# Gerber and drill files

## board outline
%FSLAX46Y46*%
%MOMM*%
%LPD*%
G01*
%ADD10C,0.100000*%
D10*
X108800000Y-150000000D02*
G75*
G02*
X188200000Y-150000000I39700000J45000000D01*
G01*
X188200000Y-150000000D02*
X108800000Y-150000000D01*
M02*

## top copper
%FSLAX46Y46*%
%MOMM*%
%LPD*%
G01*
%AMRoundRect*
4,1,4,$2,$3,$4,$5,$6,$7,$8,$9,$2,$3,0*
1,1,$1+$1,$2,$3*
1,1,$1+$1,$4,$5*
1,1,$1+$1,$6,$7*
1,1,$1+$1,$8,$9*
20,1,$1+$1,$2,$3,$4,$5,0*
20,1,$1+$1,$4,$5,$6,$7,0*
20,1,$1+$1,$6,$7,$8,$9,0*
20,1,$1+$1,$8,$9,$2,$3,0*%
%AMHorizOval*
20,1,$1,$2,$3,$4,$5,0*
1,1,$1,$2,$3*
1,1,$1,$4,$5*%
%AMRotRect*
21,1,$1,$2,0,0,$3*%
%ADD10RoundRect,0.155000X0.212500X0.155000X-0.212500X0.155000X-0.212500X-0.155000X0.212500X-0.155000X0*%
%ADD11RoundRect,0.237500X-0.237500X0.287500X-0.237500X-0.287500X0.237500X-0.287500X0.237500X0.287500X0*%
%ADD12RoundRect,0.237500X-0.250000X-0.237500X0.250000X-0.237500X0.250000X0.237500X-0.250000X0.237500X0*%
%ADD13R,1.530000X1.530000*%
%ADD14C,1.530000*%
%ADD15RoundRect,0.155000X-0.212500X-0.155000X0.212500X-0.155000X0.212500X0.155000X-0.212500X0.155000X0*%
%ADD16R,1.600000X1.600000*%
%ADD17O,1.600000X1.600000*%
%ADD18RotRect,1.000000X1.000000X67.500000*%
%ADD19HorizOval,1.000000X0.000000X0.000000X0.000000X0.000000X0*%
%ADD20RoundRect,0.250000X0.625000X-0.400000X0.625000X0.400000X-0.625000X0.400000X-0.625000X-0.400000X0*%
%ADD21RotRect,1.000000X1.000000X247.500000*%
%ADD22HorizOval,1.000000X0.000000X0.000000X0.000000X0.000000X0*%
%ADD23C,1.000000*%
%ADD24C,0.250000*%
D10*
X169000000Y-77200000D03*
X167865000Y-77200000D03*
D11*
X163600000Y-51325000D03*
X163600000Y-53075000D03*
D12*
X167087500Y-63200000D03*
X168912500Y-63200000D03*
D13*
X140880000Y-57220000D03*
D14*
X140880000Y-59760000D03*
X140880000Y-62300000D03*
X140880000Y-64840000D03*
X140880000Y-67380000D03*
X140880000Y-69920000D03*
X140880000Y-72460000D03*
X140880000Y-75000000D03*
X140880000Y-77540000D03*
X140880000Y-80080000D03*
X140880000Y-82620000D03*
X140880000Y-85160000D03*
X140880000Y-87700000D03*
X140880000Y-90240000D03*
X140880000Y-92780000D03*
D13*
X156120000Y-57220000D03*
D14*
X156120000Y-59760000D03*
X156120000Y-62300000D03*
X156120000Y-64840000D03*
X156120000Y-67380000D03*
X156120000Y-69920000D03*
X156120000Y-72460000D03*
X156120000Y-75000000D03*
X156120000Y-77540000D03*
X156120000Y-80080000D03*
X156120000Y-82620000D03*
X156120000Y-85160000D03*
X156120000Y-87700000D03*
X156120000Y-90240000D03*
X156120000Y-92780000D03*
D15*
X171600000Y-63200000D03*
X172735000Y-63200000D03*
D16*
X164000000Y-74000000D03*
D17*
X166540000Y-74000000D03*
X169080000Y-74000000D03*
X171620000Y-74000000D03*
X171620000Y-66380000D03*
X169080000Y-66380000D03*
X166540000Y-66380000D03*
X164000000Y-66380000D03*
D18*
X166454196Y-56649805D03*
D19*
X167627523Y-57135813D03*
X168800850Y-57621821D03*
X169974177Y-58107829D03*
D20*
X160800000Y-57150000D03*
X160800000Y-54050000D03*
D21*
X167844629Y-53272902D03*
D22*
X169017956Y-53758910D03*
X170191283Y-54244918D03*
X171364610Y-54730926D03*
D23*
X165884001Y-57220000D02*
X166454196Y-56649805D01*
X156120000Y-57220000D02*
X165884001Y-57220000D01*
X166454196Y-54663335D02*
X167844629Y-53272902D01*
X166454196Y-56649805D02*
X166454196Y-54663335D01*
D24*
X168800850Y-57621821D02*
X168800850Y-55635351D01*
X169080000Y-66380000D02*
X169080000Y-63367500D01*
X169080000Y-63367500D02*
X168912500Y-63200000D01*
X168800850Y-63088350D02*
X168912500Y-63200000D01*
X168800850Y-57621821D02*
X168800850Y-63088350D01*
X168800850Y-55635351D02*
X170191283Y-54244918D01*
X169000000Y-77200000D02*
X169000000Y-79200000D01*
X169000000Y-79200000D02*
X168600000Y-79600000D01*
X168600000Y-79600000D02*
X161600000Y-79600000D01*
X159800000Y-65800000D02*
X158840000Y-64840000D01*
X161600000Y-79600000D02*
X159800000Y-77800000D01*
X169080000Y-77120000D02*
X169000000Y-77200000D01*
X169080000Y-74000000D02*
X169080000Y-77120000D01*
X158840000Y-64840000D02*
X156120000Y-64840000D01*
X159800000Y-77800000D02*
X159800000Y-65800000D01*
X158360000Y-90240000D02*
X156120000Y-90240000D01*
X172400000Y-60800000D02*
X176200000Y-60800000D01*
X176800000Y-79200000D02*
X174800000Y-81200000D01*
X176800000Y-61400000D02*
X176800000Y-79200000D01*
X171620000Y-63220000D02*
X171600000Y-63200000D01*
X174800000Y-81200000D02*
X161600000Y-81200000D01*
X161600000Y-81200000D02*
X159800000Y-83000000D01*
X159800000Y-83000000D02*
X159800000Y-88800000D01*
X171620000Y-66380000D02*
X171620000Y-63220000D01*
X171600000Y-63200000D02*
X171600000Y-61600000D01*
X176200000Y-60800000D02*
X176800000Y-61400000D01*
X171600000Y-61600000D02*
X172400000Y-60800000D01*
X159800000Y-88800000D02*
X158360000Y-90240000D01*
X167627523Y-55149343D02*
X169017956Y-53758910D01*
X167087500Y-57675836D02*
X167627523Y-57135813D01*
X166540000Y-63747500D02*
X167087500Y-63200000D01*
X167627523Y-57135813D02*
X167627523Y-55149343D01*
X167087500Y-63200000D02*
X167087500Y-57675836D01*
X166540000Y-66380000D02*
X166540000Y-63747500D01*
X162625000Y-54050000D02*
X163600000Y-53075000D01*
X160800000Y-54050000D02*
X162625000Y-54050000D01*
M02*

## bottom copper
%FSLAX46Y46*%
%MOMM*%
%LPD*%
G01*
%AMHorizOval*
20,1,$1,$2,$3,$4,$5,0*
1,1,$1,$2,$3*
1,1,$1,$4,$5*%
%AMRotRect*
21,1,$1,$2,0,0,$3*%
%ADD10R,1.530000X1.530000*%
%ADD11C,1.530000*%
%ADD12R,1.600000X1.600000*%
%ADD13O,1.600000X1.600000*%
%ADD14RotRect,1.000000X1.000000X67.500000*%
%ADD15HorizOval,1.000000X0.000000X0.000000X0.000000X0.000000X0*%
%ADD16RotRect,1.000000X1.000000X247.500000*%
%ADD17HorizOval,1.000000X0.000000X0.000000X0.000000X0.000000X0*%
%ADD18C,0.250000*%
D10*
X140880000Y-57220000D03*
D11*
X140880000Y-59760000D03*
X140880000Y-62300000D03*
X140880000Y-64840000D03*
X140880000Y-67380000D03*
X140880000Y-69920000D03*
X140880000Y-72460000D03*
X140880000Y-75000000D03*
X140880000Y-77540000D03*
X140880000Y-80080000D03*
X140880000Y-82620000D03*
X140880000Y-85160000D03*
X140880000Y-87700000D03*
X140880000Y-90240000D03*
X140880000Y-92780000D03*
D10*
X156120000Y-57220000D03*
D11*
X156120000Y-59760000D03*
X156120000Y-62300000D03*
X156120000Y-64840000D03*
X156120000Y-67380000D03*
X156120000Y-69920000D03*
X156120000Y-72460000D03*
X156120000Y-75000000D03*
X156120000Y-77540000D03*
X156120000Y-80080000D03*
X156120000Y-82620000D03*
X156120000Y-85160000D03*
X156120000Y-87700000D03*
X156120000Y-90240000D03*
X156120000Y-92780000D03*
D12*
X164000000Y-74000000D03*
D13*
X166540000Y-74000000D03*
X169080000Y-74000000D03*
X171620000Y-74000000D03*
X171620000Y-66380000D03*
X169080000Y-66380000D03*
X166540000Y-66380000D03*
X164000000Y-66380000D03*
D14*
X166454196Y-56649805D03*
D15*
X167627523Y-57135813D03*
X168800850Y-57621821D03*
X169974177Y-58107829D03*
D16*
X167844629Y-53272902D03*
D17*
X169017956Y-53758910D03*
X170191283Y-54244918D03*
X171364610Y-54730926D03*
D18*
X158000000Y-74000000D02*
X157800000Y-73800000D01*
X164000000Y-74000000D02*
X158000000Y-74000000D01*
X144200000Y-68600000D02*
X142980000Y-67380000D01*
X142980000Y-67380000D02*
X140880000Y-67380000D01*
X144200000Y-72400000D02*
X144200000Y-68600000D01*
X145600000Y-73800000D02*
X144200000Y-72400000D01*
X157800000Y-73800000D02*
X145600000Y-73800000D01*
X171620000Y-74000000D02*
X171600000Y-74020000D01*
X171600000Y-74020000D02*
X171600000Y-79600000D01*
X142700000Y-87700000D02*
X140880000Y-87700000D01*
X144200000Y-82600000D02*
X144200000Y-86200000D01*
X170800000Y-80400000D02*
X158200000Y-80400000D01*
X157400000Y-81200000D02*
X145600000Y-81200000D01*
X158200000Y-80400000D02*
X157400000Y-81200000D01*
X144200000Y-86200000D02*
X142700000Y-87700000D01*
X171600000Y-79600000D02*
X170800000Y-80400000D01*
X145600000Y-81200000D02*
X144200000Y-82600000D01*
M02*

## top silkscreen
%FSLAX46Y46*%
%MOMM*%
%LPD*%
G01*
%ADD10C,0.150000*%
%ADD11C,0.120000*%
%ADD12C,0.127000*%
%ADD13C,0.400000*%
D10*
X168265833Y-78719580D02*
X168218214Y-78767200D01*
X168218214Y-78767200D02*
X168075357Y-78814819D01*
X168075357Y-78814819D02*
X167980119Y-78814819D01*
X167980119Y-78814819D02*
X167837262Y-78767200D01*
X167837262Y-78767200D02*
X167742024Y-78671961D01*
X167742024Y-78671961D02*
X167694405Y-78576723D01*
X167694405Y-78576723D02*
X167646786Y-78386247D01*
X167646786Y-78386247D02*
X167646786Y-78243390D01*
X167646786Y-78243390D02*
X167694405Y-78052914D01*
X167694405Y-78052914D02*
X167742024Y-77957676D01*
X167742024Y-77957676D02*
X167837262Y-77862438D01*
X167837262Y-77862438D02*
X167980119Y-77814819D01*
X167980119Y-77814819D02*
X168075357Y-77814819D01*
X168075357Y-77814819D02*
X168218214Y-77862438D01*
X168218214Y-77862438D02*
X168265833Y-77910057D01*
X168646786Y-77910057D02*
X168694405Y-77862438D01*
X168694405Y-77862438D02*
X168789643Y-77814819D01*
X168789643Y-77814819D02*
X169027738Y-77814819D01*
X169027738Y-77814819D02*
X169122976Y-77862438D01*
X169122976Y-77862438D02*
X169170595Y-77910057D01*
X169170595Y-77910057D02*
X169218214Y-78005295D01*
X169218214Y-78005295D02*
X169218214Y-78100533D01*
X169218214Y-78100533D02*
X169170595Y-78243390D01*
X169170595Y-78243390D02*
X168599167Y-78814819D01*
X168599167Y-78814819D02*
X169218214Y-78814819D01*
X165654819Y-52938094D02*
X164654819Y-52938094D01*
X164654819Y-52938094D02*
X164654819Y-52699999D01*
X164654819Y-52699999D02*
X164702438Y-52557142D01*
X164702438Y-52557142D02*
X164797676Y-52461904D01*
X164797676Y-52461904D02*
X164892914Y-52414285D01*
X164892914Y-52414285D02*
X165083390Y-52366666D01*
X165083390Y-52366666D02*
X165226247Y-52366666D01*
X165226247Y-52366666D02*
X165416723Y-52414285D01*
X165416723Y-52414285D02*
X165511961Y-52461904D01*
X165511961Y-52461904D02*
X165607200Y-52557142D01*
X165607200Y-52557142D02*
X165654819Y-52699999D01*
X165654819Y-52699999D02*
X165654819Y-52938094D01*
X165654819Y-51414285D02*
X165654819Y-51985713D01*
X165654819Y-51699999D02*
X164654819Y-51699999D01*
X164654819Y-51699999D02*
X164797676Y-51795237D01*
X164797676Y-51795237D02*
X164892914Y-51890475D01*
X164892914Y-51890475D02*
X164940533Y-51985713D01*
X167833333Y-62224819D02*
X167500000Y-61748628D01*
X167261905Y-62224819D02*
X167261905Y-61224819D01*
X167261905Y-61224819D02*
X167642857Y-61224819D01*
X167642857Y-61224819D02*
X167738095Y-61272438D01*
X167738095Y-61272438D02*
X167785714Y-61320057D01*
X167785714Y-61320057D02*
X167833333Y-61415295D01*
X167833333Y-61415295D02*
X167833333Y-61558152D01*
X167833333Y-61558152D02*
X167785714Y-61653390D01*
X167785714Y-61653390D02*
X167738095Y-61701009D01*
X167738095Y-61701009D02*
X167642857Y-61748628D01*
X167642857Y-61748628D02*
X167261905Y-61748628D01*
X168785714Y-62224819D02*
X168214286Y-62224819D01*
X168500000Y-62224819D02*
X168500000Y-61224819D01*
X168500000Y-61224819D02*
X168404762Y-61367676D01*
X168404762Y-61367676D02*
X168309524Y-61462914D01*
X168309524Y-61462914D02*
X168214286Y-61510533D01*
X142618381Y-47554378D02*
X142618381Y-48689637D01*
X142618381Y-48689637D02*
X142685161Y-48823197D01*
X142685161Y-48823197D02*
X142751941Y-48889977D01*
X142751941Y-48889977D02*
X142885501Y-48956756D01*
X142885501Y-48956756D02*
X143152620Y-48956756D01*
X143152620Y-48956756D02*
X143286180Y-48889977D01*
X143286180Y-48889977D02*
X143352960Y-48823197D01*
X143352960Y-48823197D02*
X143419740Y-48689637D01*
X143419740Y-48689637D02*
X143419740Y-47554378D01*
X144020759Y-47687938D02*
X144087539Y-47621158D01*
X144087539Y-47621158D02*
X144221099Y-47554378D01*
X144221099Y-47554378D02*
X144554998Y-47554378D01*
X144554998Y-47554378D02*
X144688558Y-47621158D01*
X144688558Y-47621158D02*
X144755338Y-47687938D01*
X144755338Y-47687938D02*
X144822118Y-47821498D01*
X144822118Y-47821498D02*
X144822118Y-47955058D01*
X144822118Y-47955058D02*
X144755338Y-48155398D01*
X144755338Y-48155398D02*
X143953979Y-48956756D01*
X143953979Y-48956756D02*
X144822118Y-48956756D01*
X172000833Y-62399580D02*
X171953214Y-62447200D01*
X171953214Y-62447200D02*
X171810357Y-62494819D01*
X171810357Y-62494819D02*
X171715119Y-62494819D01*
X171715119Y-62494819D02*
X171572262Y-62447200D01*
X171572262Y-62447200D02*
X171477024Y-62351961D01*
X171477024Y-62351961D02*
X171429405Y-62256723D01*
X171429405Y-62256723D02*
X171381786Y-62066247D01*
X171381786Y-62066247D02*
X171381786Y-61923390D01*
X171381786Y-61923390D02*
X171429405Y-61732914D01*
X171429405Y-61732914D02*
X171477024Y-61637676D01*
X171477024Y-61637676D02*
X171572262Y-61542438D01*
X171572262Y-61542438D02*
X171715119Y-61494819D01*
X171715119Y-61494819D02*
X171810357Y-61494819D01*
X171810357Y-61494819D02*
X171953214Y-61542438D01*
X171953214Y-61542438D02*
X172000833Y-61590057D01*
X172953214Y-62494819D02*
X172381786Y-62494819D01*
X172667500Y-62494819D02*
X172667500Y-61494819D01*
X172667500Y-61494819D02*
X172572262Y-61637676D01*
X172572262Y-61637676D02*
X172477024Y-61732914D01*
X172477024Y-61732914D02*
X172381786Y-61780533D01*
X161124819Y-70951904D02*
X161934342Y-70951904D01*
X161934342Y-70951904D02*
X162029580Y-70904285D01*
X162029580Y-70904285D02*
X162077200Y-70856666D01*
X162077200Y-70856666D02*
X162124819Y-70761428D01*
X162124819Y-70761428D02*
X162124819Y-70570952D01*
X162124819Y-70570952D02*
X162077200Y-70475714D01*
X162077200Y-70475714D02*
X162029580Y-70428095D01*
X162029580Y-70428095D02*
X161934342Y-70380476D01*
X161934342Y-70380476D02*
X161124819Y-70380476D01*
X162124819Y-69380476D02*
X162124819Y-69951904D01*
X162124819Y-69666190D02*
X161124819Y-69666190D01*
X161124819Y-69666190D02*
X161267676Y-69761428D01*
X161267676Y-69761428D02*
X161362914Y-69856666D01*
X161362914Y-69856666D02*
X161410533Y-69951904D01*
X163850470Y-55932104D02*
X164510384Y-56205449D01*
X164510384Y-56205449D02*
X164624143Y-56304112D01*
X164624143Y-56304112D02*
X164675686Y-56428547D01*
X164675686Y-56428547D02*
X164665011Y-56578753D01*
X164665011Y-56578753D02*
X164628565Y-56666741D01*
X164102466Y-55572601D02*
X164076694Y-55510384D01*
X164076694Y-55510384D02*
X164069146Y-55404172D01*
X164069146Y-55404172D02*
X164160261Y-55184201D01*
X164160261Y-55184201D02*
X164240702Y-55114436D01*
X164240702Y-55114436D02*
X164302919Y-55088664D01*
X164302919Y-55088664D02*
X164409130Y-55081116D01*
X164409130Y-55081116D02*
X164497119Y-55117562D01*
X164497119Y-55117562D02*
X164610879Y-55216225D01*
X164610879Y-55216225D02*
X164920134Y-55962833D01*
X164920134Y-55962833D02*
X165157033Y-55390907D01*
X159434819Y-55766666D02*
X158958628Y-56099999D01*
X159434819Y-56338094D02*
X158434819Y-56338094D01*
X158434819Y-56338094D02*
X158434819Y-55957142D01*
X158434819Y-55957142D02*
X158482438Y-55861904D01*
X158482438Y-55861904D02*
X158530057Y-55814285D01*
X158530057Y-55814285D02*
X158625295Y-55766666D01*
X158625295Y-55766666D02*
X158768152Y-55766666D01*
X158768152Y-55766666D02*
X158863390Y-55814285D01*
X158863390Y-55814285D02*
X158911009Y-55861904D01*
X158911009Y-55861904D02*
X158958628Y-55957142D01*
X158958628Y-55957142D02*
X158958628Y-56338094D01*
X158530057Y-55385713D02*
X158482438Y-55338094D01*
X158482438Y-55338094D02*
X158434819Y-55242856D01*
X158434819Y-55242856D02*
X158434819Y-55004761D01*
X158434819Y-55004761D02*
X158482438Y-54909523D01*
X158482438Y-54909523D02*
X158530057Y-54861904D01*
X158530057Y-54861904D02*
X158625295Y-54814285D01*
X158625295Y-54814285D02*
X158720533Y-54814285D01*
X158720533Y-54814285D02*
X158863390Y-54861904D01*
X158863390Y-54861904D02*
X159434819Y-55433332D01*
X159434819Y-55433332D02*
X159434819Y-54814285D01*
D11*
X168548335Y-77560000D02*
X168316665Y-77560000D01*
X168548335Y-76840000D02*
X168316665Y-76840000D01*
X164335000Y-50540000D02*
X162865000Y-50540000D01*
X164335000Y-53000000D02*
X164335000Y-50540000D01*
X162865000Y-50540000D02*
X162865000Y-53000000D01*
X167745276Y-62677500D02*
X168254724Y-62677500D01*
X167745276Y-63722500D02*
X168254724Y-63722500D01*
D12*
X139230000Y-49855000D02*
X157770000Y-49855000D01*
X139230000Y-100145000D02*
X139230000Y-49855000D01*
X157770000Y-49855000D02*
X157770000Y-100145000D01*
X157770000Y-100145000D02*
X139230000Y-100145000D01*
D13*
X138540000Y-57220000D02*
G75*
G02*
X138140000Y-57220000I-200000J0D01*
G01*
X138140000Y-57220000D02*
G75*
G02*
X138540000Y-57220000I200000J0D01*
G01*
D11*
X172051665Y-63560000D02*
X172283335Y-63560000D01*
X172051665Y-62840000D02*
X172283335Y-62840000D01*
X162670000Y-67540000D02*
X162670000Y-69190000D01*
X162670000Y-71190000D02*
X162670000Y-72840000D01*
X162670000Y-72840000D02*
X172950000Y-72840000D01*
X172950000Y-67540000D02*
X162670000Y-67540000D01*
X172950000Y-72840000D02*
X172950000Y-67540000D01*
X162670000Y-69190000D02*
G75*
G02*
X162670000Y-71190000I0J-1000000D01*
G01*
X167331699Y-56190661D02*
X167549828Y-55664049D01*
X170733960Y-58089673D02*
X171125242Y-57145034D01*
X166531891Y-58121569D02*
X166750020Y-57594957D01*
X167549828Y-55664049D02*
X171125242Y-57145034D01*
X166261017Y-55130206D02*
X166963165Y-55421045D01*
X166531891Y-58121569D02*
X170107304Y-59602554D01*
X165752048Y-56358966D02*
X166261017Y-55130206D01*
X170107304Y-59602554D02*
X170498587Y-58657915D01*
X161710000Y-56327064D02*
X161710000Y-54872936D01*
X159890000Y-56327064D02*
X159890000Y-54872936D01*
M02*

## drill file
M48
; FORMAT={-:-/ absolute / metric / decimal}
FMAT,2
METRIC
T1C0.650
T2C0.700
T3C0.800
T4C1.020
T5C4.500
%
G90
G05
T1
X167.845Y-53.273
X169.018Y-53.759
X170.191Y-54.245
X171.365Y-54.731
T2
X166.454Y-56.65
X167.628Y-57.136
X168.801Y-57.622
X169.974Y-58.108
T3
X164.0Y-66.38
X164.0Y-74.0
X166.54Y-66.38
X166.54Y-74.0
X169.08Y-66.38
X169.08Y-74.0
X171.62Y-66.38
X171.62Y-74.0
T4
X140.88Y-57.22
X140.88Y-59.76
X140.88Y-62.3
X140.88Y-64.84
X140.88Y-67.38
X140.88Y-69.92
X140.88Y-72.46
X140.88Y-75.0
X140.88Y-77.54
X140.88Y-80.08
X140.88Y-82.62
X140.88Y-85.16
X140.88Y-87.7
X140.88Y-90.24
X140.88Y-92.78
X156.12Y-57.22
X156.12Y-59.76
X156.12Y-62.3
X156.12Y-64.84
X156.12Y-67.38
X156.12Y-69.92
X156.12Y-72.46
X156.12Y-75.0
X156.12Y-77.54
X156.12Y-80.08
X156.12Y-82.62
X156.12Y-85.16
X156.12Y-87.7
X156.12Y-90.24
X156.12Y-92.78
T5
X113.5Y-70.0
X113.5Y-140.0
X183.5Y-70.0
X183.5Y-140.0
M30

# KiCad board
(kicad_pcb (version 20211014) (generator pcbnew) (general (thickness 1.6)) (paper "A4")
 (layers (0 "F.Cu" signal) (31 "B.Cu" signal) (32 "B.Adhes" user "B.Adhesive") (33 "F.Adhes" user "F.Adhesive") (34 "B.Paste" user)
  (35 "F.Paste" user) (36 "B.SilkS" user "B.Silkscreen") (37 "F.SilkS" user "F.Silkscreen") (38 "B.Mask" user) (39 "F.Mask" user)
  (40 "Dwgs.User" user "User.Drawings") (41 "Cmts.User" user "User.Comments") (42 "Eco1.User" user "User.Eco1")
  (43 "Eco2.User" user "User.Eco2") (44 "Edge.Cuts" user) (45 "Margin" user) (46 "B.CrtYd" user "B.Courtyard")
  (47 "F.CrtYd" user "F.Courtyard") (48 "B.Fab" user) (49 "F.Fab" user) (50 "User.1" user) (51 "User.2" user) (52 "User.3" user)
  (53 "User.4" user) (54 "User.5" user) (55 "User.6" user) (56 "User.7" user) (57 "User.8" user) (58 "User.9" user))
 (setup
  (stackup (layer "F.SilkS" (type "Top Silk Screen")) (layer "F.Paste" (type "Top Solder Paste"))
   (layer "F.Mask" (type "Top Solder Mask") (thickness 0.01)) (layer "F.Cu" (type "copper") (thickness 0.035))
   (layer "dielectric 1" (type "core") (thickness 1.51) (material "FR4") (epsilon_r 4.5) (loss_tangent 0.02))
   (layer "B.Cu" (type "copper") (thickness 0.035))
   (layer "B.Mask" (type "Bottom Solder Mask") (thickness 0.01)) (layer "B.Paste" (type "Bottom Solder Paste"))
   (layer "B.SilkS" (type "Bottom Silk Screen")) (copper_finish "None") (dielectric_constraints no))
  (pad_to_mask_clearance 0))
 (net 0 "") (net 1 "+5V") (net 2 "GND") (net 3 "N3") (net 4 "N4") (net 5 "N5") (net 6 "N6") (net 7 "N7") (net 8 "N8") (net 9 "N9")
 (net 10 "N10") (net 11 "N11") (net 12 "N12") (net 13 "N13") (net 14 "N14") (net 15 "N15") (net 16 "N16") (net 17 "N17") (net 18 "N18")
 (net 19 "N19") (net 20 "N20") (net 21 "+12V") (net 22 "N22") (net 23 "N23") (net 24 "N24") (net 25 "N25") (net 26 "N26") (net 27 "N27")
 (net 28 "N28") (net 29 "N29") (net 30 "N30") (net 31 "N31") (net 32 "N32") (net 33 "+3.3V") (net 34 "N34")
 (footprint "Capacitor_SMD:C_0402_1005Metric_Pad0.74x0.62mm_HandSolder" (layer "F.Cu") (at 168.4325 77.2 180)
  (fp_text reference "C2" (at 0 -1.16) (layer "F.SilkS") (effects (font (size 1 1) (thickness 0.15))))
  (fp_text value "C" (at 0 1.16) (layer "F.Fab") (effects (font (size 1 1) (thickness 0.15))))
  (fp_line (start -0.115835 -0.36) (end 0.115835 -0.36) (layer "F.SilkS") (width 0.12))
  (fp_line (start -0.115835 0.36) (end 0.115835 0.36) (layer "F.SilkS") (width 0.12))
  (pad "1" smd roundrect (at -0.5675 0 180) (size 0.735 0.62) (layers "F.Cu" "F.Paste" "F.Mask") (roundrect_rratio 0.25) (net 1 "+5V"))
  (pad "2" smd roundrect (at 0.5675 0 180) (size 0.735 0.62) (layers "F.Cu" "F.Paste" "F.Mask") (roundrect_rratio 0.25) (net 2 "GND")))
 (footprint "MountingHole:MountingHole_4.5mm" (layer "F.Cu") (at 183.5 140)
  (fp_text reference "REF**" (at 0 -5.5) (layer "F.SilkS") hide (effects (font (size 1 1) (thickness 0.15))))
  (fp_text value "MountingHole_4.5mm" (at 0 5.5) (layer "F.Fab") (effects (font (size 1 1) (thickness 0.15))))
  (pad "" np_thru_hole circle (at 0 0) (size 4.5 4.5) (drill 4.5) (layers *.Cu *.Mask)))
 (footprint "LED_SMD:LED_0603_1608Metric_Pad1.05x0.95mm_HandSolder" (layer "F.Cu") (at 163.6 52.2 -90)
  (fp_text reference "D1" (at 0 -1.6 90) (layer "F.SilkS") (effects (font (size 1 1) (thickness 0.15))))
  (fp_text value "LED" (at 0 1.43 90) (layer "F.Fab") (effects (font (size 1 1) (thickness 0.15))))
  (fp_line (start -1.66 -0.735) (end -1.66 0.735) (layer "F.SilkS") (width 0.12))
  (fp_line (start 0.8 -0.735) (end -1.66 -0.735) (layer "F.SilkS") (width 0.12))
  (fp_line (start -1.66 0.735) (end 0.8 0.735) (layer "F.SilkS") (width 0.12))
  (pad "1" smd roundrect (at -0.875 0 270) (size 1.05 0.95) (layers "F.Cu" "F.Paste" "F.Mask") (roundrect_rratio 0.25) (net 2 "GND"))
  (pad "2" smd roundrect (at 0.875 0 270) (size 1.05 0.95) (layers "F.Cu" "F.Paste" "F.Mask") (roundrect_rratio 0.25) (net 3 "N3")))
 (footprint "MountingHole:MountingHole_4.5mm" (layer "F.Cu") (at 113.5 140)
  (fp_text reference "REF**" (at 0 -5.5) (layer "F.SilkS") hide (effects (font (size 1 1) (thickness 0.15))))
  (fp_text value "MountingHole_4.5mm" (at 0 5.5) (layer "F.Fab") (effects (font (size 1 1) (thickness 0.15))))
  (pad "" np_thru_hole circle (at 0 0) (size 4.5 4.5) (drill 4.5) (layers F&B.Cu *.Mask)))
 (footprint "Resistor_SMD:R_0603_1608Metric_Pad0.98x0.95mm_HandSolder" (layer "F.Cu") (at 168 63.2)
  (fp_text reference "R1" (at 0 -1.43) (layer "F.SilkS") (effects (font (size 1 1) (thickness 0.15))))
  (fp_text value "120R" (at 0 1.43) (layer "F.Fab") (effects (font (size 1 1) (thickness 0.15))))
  (fp_line (start -0.254724 -0.5225) (end 0.254724 -0.5225) (layer "F.SilkS") (width 0.12))
  (fp_line (start -0.254724 0.5225) (end 0.254724 0.5225) (layer "F.SilkS") (width 0.12))
  (pad "1" smd roundrect (at -0.9125 0) (size 0.975 0.95) (layers "F.Cu" "F.Paste" "F.Mask") (roundrect_rratio 0.25) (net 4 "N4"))
  (pad "2" smd roundrect (at 0.9125 0) (size 0.975 0.95) (layers "F.Cu" "F.Paste" "F.Mask") (roundrect_rratio 0.25) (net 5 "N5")))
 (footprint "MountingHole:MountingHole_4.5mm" (layer "F.Cu") (at 183.5 70)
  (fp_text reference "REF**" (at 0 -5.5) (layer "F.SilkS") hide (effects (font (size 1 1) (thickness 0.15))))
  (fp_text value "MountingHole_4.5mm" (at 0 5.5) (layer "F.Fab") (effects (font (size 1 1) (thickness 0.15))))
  (pad "" np_thru_hole circle (at 0 0) (size 4.5 4.5) (drill 4.5) (layers F&B.Cu *.Mask)))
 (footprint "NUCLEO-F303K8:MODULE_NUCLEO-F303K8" (layer "F.Cu") (at 148.5 75)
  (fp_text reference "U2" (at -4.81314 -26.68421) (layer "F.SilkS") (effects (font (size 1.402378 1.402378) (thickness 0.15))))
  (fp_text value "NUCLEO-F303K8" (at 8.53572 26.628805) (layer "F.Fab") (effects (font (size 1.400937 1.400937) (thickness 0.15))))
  (fp_line (start -9.27 -25.145) (end 9.27 -25.145) (layer "F.SilkS") (width 0.127))
  (fp_line (start -9.27 25.145) (end -9.27 -25.145) (layer "F.SilkS") (width 0.127))
  (fp_line (start 9.27 -25.145) (end 9.27 25.145) (layer "F.SilkS") (width 0.127))
  (fp_line (start 9.27 25.145) (end -9.27 25.145) (layer "F.SilkS") (width 0.127))
  (fp_circle (center -10.16 -17.78) (end -9.96 -17.78) (layer "F.SilkS") (width 0.4) (fill none))
  (pad "3_1" thru_hole rect locked (at -7.62 -17.78) (size 1.53 1.53) (drill 1.02) (layers *.Cu *.Mask) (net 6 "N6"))
  (pad "3_2" thru_hole circle locked (at -7.62 -15.24) (size 1.53 1.53) (drill 1.02) (layers *.Cu *.Mask) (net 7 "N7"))
  (pad "3_3" thru_hole circle locked (at -7.62 -12.7) (size 1.53 1.53) (drill 1.02) (layers *.Cu *.Mask) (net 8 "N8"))
  (pad "3_4" thru_hole circle locked (at -7.62 -10.16) (size 1.53 1.53) (drill 1.02) (layers *.Cu *.Mask) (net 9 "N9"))
  (pad "3_5" thru_hole circle locked (at -7.62 -7.62) (size 1.53 1.53) (drill 1.02) (layers *.Cu *.Mask) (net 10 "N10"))
  (pad "3_6" thru_hole circle locked (at -7.62 -5.08) (size 1.53 1.53) (drill 1.02) (layers *.Cu *.Mask) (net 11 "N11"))
  (pad "3_7" thru_hole circle locked (at -7.62 -2.54) (size 1.53 1.53) (drill 1.02) (layers *.Cu *.Mask) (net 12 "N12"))
  (pad "3_8" thru_hole circle locked (at -7.62 0) (size 1.53 1.53) (drill 1.02) (layers *.Cu *.Mask) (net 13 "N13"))
  (pad "3_9" thru_hole circle locked (at -7.62 2.54) (size 1.53 1.53) (drill 1.02) (layers *.Cu *.Mask) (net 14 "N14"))
  (pad "3_10" thru_hole circle locked (at -7.62 5.08) (size 1.53 1.53) (drill 1.02) (layers *.Cu *.Mask) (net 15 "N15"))
  (pad "3_11" thru_hole circle locked (at -7.62 7.62) (size 1.53 1.53) (drill 1.02) (layers *.Cu *.Mask) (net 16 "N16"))
  (pad "3_12" thru_hole circle locked (at -7.62 10.16) (size 1.53 1.53) (drill 1.02) (layers *.Cu *.Mask) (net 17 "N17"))
  (pad "3_13" thru_hole circle locked (at -7.62 12.7) (size 1.53 1.53) (drill 1.02) (layers *.Cu *.Mask) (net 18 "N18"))
  (pad "3_14" thru_hole circle locked (at -7.62 15.24) (size 1.53 1.53) (drill 1.02) (layers *.Cu *.Mask) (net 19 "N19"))
  (pad "3_15" thru_hole circle locked (at -7.62 17.78) (size 1.53 1.53) (drill 1.02) (layers *.Cu *.Mask) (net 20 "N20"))
  (pad "4_1" thru_hole rect locked (at 7.62 -17.78) (size 1.53 1.53) (drill 1.02) (layers *.Cu *.Mask) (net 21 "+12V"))
  (pad "4_2" thru_hole circle locked (at 7.62 -15.24) (size 1.53 1.53) (drill 1.02) (layers *.Cu *.Mask) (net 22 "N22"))
  (pad "4_3" thru_hole circle locked (at 7.62 -12.7) (size 1.53 1.53) (drill 1.02) (layers *.Cu *.Mask) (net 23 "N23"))
  (pad "4_4" thru_hole circle locked (at 7.62 -10.16) (size 1.53 1.53) (drill 1.02) (layers *.Cu *.Mask) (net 1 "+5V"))
  (pad "4_5" thru_hole circle locked (at 7.62 -7.62) (size 1.53 1.53) (drill 1.02) (layers *.Cu *.Mask) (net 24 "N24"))
  (pad "4_6" thru_hole circle locked (at 7.62 -5.08) (size 1.53 1.53) (drill 1.02) (layers *.Cu *.Mask) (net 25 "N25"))
  (pad "4_7" thru_hole circle locked (at 7.62 -2.54) (size 1.53 1.53) (drill 1.02) (layers *.Cu *.Mask) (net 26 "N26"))
  (pad "4_8" thru_hole circle locked (at 7.62 0) (size 1.53 1.53) (drill 1.02) (layers *.Cu *.Mask) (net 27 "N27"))
  (pad "4_9" thru_hole circle locked (at 7.62 2.54) (size 1.53 1.53) (drill 1.02) (layers *.Cu *.Mask) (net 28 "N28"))
  (pad "4_10" thru_hole circle locked (at 7.62 5.08) (size 1.53 1.53) (drill 1.02) (layers *.Cu *.Mask) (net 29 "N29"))
  (pad "4_11" thru_hole circle locked (at 7.62 7.62) (size 1.53 1.53) (drill 1.02) (layers *.Cu *.Mask) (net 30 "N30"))
  (pad "4_12" thru_hole circle locked (at 7.62 10.16) (size 1.53 1.53) (drill 1.02) (layers *.Cu *.Mask) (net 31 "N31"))
  (pad "4_13" thru_hole circle locked (at 7.62 12.7) (size 1.53 1.53) (drill 1.02) (layers *.Cu *.Mask) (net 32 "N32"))
  (pad "4_14" thru_hole circle locked (at 7.62 15.24) (size 1.53 1.53) (drill 1.02) (layers *.Cu *.Mask) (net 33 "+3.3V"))
  (pad "4_15" thru_hole circle locked (at 7.62 17.78) (size 1.53 1.53) (drill 1.02) (layers *.Cu *.Mask) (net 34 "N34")))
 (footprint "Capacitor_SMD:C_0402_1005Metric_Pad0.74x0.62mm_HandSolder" (layer "F.Cu") (at 172.1675 63.2)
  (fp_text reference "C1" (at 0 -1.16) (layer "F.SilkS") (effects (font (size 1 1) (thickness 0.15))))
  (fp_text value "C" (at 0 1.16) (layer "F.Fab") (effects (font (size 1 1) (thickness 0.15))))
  (fp_line (start -0.115835 0.36) (end 0.115835 0.36) (layer "F.SilkS") (width 0.12))
  (fp_line (start -0.115835 -0.36) (end 0.115835 -0.36) (layer "F.SilkS") (width 0.12))
  (pad "1" smd roundrect (at -0.5675 0) (size 0.735 0.62) (layers "F.Cu" "F.Paste" "F.Mask") (roundrect_rratio 0.25) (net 33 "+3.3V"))
  (pad "2" smd roundrect (at 0.5675 0) (size 0.735 0.62) (layers "F.Cu" "F.Paste" "F.Mask") (roundrect_rratio 0.25) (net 2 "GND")))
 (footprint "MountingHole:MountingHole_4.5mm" (layer "F.Cu") (at 113.5 70)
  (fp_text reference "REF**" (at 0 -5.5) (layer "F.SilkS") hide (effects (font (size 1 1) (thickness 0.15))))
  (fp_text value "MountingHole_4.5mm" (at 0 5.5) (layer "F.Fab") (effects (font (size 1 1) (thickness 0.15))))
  (pad "" np_thru_hole circle (at 0 0) (size 4.5 4.5) (drill 4.5) (layers F&B.Cu *.Mask)))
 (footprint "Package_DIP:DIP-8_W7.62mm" (layer "F.Cu") (at 164 74 90)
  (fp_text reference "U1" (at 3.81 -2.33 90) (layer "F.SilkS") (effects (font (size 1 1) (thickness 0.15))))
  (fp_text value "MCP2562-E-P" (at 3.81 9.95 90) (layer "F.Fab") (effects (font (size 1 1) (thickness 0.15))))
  (fp_line (start 6.46 -1.33) (end 4.81 -1.33) (layer "F.SilkS") (width 0.12))
  (fp_line (start 2.81 -1.33) (end 1.16 -1.33) (layer "F.SilkS") (width 0.12))
  (fp_line (start 1.16 -1.33) (end 1.16 8.95) (layer "F.SilkS") (width 0.12))
  (fp_line (start 6.46 8.95) (end 6.46 -1.33) (layer "F.SilkS") (width 0.12))
  (fp_line (start 1.16 8.95) (end 6.46 8.95) (layer "F.SilkS") (width 0.12))
  (fp_arc (start 4.81 -1.33) (mid 3.81 -0.33) (end 2.81 -1.33) (layer "F.SilkS") (width 0.12))
  (pad "1" thru_hole rect (at 0 0 90) (size 1.6 1.6) (drill 0.8) (layers *.Cu *.Mask) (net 10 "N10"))
  (pad "2" thru_hole oval (at 0 2.54 90) (size 1.6 1.6) (drill 0.8) (layers *.Cu *.Mask) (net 2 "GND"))
  (pad "3" thru_hole oval (at 0 5.08 90) (size 1.6 1.6) (drill 0.8) (layers *.Cu *.Mask) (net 1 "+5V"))
  (pad "4" thru_hole oval (at 0 7.62 90) (size 1.6 1.6) (drill 0.8) (layers *.Cu *.Mask) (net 18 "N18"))
  (pad "5" thru_hole oval (at 7.62 7.62 90) (size 1.6 1.6) (drill 0.8) (layers *.Cu *.Mask) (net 33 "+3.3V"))
  (pad "6" thru_hole oval (at 7.62 5.08 90) (size 1.6 1.6) (drill 0.8) (layers *.Cu *.Mask) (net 5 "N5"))
  (pad "7" thru_hole oval (at 7.62 2.54 90) (size 1.6 1.6) (drill 0.8) (layers *.Cu *.Mask) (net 4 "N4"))
  (pad "8" thru_hole oval (at 7.62 0 90) (size 1.6 1.6) (drill 0.8) (layers *.Cu *.Mask) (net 2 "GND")))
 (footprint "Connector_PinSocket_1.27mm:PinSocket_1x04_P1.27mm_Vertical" (layer "F.Cu") (at 166.454196 56.649805 67.5)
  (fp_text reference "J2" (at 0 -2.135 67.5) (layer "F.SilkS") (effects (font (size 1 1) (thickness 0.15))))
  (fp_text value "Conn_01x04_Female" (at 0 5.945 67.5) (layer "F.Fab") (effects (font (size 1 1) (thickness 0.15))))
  (fp_line (start 0.76 0.635) (end 1.33 0.635) (layer "F.SilkS") (width 0.12))
  (fp_line (start 0.30753 4.505) (end 1.33 4.505) (layer "F.SilkS") (width 0.12))
  (fp_line (start -1.33 0.635) (end -0.76 0.635) (layer "F.SilkS") (width 0.12))
  (fp_line (start 1.33 0.635) (end 1.33 4.505) (layer "F.SilkS") (width 0.12))
  (fp_line (start 1.33 -0.76) (end 1.33 0) (layer "F.SilkS") (width 0.12))
  (fp_line (start -1.33 0.635) (end -1.33 4.505) (layer "F.SilkS") (width 0.12))
  (fp_line (start 0 -0.76) (end 1.33 -0.76) (layer "F.SilkS") (width 0.12))
  (fp_line (start -1.33 4.505) (end -0.30753 4.505) (layer "F.SilkS") (width 0.12))
  (pad "1" thru_hole rect (at 0 0 67.5) (size 1 1) (drill 0.7) (layers *.Cu *.Mask) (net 21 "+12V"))
  (pad "2" thru_hole oval (at 0 1.27 67.5) (size 1 1) (drill 0.7) (layers *.Cu *.Mask) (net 4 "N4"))
  (pad "3" thru_hole oval (at 0 2.54 67.5) (size 1 1) (drill 0.7) (layers *.Cu *.Mask) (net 5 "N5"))
  (pad "4" thru_hole oval (at 0 3.81 67.5) (size 1 1) (drill 0.7) (layers *.Cu *.Mask) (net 2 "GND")))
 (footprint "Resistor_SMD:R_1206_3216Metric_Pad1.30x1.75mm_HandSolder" (layer "F.Cu") (at 160.8 55.6 90)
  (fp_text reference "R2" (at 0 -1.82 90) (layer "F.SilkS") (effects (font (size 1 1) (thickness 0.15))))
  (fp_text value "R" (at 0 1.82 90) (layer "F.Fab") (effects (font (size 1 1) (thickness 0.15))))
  (fp_line (start -0.727064 0.91) (end 0.727064 0.91) (layer "F.SilkS") (width 0.12))
  (fp_line (start -0.727064 -0.91) (end 0.727064 -0.91) (layer "F.SilkS") (width 0.12))
  (pad "1" smd roundrect (at -1.55 0 90) (size 1.3 1.75) (layers "F.Cu" "F.Paste" "F.Mask") (roundrect_rratio 0.192308) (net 21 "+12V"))
  (pad "2" smd roundrect (at 1.55 0 90) (size 1.3 1.75) (layers "F.Cu" "F.Paste" "F.Mask") (roundrect_rratio 0.192308) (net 3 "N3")))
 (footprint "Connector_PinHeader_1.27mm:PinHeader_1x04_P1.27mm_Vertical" (layer "B.Cu") (at 167.844629 53.272902 -112.5)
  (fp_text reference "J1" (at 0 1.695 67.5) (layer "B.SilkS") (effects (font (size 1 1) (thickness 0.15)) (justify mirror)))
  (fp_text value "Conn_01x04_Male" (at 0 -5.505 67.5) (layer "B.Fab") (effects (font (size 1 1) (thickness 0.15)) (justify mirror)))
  (pad "1" thru_hole rect (at 0 0 247.5) (size 1 1) (drill 0.65) (layers *.Cu *.Mask) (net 21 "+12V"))
  (pad "2" thru_hole oval (at 0 -1.27 247.5) (size 1 1) (drill 0.65) (layers *.Cu *.Mask) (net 4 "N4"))
  (pad "3" thru_hole oval (at 0 -2.54 247.5) (size 1 1) (drill 0.65) (layers *.Cu *.Mask) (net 5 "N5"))
  (pad "4" thru_hole oval (at 0 -3.81 247.5) (size 1 1) (drill 0.65) (layers *.Cu *.Mask) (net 2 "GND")))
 (gr_arc locked (start 108.8 150) (mid 148.5 44.990917) (end 188.2 150) (layer "Edge.Cuts") (width 0.1))
 (gr_line locked (start 188.2 150) (end 108.8 150) (layer "Edge.Cuts") (width 0.1))
 (segment (start 165.884001 57.22) (end 166.454196 56.649805) (width 1) (layer "F.Cu") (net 21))
 (segment (start 156.12 57.22) (end 165.884001 57.22) (width 1) (layer "F.Cu") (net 21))
 (segment (start 166.454196 54.663335) (end 167.844629 53.272902) (width 1) (layer "F.Cu") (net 21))
 (segment (start 166.454196 56.649805) (end 166.454196 54.663335) (width 1) (layer "F.Cu") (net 21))
 (segment (start 168.80085 57.621821) (end 168.80085 55.635351) (width 0.25) (layer "F.Cu") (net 5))
 (segment (start 169.08 66.38) (end 169.08 63.3675) (width 0.25) (layer "F.Cu") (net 5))
 (segment (start 169.08 63.3675) (end 168.9125 63.2) (width 0.25) (layer "F.Cu") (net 5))
 (segment (start 168.80085 63.08835) (end 168.9125 63.2) (width 0.25) (layer "F.Cu") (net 5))
 (segment (start 168.80085 57.621821) (end 168.80085 63.08835) (width 0.25) (layer "F.Cu") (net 5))
 (segment (start 168.80085 55.635351) (end 170.191283 54.244918) (width 0.25) (layer "F.Cu") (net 5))
 (segment (start 158 74) (end 157.8 73.8) (width 0.25) (layer "B.Cu") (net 10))
 (segment (start 164 74) (end 158 74) (width 0.25) (layer "B.Cu") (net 10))
 (segment (start 144.2 68.6) (end 142.98 67.38) (width 0.25) (layer "B.Cu") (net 10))
 (segment (start 142.98 67.38) (end 140.88 67.38) (width 0.25) (layer "B.Cu") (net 10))
 (segment (start 144.2 72.4) (end 144.2 68.6) (width 0.25) (layer "B.Cu") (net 10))
 (segment (start 145.6 73.8) (end 144.2 72.4) (width 0.25) (layer "B.Cu") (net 10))
 (segment (start 157.8 73.8) (end 145.6 73.8) (width 0.25) (layer "B.Cu") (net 10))
 (segment (start 169 77.2) (end 169 79.2) (width 0.25) (layer "F.Cu") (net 1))
 (segment (start 169 79.2) (end 168.6 79.6) (width 0.25) (layer "F.Cu") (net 1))
 (segment (start 168.6 79.6) (end 161.6 79.6) (width 0.25) (layer "F.Cu") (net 1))
 (segment (start 159.8 65.8) (end 158.84 64.84) (width 0.25) (layer "F.Cu") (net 1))
 (segment (start 161.6 79.6) (end 159.8 77.8) (width 0.25) (layer "F.Cu") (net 1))
 (segment (start 169.08 77.12) (end 169 77.2) (width 0.25) (layer "F.Cu") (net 1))
 (segment (start 169.08 74) (end 169.08 77.12) (width 0.25) (layer "F.Cu") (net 1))
 (segment (start 158.84 64.84) (end 156.12 64.84) (width 0.25) (layer "F.Cu") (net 1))
 (segment (start 159.8 77.8) (end 159.8 65.8) (width 0.25) (layer "F.Cu") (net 1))
 (segment (start 171.62 74) (end 171.6 74.02) (width 0.25) (layer "B.Cu") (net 18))
 (segment (start 171.6 74.02) (end 171.6 79.6) (width 0.25) (layer "B.Cu") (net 18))
 (segment (start 142.7 87.7) (end 140.88 87.7) (width 0.25) (layer "B.Cu") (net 18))
 (segment (start 144.2 82.6) (end 144.2 86.2) (width 0.25) (layer "B.Cu") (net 18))
 (segment (start 170.8 80.4) (end 158.2 80.4) (width 0.25) (layer "B.Cu") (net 18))
 (segment (start 157.4 81.2) (end 145.6 81.2) (width 0.25) (layer "B.Cu") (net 18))
 (segment (start 158.2 80.4) (end 157.4 81.2) (width 0.25) (layer "B.Cu") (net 18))
 (segment (start 144.2 86.2) (end 142.7 87.7) (width 0.25) (layer "B.Cu") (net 18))
 (segment (start 171.6 79.6) (end 170.8 80.4) (width 0.25) (layer "B.Cu") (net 18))
 (segment (start 145.6 81.2) (end 144.2 82.6) (width 0.25) (layer "B.Cu") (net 18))
 (segment (start 158.36 90.24) (end 156.12 90.24) (width 0.25) (layer "F.Cu") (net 33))
 (segment (start 172.4 60.8) (end 176.2 60.8) (width 0.25) (layer "F.Cu") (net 33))
 (segment (start 176.8 79.2) (end 174.8 81.2) (width 0.25) (layer "F.Cu") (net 33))
 (segment (start 176.8 61.4) (end 176.8 79.2) (width 0.25) (layer "F.Cu") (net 33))
 (segment (start 171.62 63.22) (end 171.6 63.2) (width 0.25) (layer "F.Cu") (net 33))
 (segment (start 174.8 81.2) (end 161.6 81.2) (width 0.25) (layer "F.Cu") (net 33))
 (segment (start 161.6 81.2) (end 159.8 83) (width 0.25) (layer "F.Cu") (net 33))
 (segment (start 159.8 83) (end 159.8 88.8) (width 0.25) (layer "F.Cu") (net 33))
 (segment (start 171.62 66.38) (end 171.62 63.22) (width 0.25) (layer "F.Cu") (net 33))
 (segment (start 171.6 63.2) (end 171.6 61.6) (width 0.25) (layer "F.Cu") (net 33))
 (segment (start 176.2 60.8) (end 176.8 61.4) (width 0.25) (layer "F.Cu") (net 33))
 (segment (start 171.6 61.6) (end 172.4 60.8) (width 0.25) (layer "F.Cu") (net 33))
 (segment (start 159.8 88.8) (end 158.36 90.24) (width 0.25) (layer "F.Cu") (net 33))
 (segment (start 167.627523 55.149343) (end 169.017956 53.75891) (width 0.25) (layer "F.Cu") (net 4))
 (segment (start 167.0875 57.675836) (end 167.627523 57.135813) (width 0.25) (layer "F.Cu") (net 4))
 (segment (start 166.54 63.7475) (end 167.0875 63.2) (width 0.25) (layer "F.Cu") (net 4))
 (segment (start 167.627523 57.135813) (end 167.627523 55.149343) (width 0.25) (layer "F.Cu") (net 4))
 (segment (start 167.0875 63.2) (end 167.0875 57.675836) (width 0.25) (layer "F.Cu") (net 4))
 (segment (start 166.54 66.38) (end 166.54 63.7475) (width 0.25) (layer "F.Cu") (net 4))
 (segment (start 162.625 54.05) (end 163.6 53.075) (width 0.25) (layer "F.Cu") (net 3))
 (segment (start 160.8 54.05) (end 162.625 54.05) (width 0.25) (layer "F.Cu") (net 3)))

